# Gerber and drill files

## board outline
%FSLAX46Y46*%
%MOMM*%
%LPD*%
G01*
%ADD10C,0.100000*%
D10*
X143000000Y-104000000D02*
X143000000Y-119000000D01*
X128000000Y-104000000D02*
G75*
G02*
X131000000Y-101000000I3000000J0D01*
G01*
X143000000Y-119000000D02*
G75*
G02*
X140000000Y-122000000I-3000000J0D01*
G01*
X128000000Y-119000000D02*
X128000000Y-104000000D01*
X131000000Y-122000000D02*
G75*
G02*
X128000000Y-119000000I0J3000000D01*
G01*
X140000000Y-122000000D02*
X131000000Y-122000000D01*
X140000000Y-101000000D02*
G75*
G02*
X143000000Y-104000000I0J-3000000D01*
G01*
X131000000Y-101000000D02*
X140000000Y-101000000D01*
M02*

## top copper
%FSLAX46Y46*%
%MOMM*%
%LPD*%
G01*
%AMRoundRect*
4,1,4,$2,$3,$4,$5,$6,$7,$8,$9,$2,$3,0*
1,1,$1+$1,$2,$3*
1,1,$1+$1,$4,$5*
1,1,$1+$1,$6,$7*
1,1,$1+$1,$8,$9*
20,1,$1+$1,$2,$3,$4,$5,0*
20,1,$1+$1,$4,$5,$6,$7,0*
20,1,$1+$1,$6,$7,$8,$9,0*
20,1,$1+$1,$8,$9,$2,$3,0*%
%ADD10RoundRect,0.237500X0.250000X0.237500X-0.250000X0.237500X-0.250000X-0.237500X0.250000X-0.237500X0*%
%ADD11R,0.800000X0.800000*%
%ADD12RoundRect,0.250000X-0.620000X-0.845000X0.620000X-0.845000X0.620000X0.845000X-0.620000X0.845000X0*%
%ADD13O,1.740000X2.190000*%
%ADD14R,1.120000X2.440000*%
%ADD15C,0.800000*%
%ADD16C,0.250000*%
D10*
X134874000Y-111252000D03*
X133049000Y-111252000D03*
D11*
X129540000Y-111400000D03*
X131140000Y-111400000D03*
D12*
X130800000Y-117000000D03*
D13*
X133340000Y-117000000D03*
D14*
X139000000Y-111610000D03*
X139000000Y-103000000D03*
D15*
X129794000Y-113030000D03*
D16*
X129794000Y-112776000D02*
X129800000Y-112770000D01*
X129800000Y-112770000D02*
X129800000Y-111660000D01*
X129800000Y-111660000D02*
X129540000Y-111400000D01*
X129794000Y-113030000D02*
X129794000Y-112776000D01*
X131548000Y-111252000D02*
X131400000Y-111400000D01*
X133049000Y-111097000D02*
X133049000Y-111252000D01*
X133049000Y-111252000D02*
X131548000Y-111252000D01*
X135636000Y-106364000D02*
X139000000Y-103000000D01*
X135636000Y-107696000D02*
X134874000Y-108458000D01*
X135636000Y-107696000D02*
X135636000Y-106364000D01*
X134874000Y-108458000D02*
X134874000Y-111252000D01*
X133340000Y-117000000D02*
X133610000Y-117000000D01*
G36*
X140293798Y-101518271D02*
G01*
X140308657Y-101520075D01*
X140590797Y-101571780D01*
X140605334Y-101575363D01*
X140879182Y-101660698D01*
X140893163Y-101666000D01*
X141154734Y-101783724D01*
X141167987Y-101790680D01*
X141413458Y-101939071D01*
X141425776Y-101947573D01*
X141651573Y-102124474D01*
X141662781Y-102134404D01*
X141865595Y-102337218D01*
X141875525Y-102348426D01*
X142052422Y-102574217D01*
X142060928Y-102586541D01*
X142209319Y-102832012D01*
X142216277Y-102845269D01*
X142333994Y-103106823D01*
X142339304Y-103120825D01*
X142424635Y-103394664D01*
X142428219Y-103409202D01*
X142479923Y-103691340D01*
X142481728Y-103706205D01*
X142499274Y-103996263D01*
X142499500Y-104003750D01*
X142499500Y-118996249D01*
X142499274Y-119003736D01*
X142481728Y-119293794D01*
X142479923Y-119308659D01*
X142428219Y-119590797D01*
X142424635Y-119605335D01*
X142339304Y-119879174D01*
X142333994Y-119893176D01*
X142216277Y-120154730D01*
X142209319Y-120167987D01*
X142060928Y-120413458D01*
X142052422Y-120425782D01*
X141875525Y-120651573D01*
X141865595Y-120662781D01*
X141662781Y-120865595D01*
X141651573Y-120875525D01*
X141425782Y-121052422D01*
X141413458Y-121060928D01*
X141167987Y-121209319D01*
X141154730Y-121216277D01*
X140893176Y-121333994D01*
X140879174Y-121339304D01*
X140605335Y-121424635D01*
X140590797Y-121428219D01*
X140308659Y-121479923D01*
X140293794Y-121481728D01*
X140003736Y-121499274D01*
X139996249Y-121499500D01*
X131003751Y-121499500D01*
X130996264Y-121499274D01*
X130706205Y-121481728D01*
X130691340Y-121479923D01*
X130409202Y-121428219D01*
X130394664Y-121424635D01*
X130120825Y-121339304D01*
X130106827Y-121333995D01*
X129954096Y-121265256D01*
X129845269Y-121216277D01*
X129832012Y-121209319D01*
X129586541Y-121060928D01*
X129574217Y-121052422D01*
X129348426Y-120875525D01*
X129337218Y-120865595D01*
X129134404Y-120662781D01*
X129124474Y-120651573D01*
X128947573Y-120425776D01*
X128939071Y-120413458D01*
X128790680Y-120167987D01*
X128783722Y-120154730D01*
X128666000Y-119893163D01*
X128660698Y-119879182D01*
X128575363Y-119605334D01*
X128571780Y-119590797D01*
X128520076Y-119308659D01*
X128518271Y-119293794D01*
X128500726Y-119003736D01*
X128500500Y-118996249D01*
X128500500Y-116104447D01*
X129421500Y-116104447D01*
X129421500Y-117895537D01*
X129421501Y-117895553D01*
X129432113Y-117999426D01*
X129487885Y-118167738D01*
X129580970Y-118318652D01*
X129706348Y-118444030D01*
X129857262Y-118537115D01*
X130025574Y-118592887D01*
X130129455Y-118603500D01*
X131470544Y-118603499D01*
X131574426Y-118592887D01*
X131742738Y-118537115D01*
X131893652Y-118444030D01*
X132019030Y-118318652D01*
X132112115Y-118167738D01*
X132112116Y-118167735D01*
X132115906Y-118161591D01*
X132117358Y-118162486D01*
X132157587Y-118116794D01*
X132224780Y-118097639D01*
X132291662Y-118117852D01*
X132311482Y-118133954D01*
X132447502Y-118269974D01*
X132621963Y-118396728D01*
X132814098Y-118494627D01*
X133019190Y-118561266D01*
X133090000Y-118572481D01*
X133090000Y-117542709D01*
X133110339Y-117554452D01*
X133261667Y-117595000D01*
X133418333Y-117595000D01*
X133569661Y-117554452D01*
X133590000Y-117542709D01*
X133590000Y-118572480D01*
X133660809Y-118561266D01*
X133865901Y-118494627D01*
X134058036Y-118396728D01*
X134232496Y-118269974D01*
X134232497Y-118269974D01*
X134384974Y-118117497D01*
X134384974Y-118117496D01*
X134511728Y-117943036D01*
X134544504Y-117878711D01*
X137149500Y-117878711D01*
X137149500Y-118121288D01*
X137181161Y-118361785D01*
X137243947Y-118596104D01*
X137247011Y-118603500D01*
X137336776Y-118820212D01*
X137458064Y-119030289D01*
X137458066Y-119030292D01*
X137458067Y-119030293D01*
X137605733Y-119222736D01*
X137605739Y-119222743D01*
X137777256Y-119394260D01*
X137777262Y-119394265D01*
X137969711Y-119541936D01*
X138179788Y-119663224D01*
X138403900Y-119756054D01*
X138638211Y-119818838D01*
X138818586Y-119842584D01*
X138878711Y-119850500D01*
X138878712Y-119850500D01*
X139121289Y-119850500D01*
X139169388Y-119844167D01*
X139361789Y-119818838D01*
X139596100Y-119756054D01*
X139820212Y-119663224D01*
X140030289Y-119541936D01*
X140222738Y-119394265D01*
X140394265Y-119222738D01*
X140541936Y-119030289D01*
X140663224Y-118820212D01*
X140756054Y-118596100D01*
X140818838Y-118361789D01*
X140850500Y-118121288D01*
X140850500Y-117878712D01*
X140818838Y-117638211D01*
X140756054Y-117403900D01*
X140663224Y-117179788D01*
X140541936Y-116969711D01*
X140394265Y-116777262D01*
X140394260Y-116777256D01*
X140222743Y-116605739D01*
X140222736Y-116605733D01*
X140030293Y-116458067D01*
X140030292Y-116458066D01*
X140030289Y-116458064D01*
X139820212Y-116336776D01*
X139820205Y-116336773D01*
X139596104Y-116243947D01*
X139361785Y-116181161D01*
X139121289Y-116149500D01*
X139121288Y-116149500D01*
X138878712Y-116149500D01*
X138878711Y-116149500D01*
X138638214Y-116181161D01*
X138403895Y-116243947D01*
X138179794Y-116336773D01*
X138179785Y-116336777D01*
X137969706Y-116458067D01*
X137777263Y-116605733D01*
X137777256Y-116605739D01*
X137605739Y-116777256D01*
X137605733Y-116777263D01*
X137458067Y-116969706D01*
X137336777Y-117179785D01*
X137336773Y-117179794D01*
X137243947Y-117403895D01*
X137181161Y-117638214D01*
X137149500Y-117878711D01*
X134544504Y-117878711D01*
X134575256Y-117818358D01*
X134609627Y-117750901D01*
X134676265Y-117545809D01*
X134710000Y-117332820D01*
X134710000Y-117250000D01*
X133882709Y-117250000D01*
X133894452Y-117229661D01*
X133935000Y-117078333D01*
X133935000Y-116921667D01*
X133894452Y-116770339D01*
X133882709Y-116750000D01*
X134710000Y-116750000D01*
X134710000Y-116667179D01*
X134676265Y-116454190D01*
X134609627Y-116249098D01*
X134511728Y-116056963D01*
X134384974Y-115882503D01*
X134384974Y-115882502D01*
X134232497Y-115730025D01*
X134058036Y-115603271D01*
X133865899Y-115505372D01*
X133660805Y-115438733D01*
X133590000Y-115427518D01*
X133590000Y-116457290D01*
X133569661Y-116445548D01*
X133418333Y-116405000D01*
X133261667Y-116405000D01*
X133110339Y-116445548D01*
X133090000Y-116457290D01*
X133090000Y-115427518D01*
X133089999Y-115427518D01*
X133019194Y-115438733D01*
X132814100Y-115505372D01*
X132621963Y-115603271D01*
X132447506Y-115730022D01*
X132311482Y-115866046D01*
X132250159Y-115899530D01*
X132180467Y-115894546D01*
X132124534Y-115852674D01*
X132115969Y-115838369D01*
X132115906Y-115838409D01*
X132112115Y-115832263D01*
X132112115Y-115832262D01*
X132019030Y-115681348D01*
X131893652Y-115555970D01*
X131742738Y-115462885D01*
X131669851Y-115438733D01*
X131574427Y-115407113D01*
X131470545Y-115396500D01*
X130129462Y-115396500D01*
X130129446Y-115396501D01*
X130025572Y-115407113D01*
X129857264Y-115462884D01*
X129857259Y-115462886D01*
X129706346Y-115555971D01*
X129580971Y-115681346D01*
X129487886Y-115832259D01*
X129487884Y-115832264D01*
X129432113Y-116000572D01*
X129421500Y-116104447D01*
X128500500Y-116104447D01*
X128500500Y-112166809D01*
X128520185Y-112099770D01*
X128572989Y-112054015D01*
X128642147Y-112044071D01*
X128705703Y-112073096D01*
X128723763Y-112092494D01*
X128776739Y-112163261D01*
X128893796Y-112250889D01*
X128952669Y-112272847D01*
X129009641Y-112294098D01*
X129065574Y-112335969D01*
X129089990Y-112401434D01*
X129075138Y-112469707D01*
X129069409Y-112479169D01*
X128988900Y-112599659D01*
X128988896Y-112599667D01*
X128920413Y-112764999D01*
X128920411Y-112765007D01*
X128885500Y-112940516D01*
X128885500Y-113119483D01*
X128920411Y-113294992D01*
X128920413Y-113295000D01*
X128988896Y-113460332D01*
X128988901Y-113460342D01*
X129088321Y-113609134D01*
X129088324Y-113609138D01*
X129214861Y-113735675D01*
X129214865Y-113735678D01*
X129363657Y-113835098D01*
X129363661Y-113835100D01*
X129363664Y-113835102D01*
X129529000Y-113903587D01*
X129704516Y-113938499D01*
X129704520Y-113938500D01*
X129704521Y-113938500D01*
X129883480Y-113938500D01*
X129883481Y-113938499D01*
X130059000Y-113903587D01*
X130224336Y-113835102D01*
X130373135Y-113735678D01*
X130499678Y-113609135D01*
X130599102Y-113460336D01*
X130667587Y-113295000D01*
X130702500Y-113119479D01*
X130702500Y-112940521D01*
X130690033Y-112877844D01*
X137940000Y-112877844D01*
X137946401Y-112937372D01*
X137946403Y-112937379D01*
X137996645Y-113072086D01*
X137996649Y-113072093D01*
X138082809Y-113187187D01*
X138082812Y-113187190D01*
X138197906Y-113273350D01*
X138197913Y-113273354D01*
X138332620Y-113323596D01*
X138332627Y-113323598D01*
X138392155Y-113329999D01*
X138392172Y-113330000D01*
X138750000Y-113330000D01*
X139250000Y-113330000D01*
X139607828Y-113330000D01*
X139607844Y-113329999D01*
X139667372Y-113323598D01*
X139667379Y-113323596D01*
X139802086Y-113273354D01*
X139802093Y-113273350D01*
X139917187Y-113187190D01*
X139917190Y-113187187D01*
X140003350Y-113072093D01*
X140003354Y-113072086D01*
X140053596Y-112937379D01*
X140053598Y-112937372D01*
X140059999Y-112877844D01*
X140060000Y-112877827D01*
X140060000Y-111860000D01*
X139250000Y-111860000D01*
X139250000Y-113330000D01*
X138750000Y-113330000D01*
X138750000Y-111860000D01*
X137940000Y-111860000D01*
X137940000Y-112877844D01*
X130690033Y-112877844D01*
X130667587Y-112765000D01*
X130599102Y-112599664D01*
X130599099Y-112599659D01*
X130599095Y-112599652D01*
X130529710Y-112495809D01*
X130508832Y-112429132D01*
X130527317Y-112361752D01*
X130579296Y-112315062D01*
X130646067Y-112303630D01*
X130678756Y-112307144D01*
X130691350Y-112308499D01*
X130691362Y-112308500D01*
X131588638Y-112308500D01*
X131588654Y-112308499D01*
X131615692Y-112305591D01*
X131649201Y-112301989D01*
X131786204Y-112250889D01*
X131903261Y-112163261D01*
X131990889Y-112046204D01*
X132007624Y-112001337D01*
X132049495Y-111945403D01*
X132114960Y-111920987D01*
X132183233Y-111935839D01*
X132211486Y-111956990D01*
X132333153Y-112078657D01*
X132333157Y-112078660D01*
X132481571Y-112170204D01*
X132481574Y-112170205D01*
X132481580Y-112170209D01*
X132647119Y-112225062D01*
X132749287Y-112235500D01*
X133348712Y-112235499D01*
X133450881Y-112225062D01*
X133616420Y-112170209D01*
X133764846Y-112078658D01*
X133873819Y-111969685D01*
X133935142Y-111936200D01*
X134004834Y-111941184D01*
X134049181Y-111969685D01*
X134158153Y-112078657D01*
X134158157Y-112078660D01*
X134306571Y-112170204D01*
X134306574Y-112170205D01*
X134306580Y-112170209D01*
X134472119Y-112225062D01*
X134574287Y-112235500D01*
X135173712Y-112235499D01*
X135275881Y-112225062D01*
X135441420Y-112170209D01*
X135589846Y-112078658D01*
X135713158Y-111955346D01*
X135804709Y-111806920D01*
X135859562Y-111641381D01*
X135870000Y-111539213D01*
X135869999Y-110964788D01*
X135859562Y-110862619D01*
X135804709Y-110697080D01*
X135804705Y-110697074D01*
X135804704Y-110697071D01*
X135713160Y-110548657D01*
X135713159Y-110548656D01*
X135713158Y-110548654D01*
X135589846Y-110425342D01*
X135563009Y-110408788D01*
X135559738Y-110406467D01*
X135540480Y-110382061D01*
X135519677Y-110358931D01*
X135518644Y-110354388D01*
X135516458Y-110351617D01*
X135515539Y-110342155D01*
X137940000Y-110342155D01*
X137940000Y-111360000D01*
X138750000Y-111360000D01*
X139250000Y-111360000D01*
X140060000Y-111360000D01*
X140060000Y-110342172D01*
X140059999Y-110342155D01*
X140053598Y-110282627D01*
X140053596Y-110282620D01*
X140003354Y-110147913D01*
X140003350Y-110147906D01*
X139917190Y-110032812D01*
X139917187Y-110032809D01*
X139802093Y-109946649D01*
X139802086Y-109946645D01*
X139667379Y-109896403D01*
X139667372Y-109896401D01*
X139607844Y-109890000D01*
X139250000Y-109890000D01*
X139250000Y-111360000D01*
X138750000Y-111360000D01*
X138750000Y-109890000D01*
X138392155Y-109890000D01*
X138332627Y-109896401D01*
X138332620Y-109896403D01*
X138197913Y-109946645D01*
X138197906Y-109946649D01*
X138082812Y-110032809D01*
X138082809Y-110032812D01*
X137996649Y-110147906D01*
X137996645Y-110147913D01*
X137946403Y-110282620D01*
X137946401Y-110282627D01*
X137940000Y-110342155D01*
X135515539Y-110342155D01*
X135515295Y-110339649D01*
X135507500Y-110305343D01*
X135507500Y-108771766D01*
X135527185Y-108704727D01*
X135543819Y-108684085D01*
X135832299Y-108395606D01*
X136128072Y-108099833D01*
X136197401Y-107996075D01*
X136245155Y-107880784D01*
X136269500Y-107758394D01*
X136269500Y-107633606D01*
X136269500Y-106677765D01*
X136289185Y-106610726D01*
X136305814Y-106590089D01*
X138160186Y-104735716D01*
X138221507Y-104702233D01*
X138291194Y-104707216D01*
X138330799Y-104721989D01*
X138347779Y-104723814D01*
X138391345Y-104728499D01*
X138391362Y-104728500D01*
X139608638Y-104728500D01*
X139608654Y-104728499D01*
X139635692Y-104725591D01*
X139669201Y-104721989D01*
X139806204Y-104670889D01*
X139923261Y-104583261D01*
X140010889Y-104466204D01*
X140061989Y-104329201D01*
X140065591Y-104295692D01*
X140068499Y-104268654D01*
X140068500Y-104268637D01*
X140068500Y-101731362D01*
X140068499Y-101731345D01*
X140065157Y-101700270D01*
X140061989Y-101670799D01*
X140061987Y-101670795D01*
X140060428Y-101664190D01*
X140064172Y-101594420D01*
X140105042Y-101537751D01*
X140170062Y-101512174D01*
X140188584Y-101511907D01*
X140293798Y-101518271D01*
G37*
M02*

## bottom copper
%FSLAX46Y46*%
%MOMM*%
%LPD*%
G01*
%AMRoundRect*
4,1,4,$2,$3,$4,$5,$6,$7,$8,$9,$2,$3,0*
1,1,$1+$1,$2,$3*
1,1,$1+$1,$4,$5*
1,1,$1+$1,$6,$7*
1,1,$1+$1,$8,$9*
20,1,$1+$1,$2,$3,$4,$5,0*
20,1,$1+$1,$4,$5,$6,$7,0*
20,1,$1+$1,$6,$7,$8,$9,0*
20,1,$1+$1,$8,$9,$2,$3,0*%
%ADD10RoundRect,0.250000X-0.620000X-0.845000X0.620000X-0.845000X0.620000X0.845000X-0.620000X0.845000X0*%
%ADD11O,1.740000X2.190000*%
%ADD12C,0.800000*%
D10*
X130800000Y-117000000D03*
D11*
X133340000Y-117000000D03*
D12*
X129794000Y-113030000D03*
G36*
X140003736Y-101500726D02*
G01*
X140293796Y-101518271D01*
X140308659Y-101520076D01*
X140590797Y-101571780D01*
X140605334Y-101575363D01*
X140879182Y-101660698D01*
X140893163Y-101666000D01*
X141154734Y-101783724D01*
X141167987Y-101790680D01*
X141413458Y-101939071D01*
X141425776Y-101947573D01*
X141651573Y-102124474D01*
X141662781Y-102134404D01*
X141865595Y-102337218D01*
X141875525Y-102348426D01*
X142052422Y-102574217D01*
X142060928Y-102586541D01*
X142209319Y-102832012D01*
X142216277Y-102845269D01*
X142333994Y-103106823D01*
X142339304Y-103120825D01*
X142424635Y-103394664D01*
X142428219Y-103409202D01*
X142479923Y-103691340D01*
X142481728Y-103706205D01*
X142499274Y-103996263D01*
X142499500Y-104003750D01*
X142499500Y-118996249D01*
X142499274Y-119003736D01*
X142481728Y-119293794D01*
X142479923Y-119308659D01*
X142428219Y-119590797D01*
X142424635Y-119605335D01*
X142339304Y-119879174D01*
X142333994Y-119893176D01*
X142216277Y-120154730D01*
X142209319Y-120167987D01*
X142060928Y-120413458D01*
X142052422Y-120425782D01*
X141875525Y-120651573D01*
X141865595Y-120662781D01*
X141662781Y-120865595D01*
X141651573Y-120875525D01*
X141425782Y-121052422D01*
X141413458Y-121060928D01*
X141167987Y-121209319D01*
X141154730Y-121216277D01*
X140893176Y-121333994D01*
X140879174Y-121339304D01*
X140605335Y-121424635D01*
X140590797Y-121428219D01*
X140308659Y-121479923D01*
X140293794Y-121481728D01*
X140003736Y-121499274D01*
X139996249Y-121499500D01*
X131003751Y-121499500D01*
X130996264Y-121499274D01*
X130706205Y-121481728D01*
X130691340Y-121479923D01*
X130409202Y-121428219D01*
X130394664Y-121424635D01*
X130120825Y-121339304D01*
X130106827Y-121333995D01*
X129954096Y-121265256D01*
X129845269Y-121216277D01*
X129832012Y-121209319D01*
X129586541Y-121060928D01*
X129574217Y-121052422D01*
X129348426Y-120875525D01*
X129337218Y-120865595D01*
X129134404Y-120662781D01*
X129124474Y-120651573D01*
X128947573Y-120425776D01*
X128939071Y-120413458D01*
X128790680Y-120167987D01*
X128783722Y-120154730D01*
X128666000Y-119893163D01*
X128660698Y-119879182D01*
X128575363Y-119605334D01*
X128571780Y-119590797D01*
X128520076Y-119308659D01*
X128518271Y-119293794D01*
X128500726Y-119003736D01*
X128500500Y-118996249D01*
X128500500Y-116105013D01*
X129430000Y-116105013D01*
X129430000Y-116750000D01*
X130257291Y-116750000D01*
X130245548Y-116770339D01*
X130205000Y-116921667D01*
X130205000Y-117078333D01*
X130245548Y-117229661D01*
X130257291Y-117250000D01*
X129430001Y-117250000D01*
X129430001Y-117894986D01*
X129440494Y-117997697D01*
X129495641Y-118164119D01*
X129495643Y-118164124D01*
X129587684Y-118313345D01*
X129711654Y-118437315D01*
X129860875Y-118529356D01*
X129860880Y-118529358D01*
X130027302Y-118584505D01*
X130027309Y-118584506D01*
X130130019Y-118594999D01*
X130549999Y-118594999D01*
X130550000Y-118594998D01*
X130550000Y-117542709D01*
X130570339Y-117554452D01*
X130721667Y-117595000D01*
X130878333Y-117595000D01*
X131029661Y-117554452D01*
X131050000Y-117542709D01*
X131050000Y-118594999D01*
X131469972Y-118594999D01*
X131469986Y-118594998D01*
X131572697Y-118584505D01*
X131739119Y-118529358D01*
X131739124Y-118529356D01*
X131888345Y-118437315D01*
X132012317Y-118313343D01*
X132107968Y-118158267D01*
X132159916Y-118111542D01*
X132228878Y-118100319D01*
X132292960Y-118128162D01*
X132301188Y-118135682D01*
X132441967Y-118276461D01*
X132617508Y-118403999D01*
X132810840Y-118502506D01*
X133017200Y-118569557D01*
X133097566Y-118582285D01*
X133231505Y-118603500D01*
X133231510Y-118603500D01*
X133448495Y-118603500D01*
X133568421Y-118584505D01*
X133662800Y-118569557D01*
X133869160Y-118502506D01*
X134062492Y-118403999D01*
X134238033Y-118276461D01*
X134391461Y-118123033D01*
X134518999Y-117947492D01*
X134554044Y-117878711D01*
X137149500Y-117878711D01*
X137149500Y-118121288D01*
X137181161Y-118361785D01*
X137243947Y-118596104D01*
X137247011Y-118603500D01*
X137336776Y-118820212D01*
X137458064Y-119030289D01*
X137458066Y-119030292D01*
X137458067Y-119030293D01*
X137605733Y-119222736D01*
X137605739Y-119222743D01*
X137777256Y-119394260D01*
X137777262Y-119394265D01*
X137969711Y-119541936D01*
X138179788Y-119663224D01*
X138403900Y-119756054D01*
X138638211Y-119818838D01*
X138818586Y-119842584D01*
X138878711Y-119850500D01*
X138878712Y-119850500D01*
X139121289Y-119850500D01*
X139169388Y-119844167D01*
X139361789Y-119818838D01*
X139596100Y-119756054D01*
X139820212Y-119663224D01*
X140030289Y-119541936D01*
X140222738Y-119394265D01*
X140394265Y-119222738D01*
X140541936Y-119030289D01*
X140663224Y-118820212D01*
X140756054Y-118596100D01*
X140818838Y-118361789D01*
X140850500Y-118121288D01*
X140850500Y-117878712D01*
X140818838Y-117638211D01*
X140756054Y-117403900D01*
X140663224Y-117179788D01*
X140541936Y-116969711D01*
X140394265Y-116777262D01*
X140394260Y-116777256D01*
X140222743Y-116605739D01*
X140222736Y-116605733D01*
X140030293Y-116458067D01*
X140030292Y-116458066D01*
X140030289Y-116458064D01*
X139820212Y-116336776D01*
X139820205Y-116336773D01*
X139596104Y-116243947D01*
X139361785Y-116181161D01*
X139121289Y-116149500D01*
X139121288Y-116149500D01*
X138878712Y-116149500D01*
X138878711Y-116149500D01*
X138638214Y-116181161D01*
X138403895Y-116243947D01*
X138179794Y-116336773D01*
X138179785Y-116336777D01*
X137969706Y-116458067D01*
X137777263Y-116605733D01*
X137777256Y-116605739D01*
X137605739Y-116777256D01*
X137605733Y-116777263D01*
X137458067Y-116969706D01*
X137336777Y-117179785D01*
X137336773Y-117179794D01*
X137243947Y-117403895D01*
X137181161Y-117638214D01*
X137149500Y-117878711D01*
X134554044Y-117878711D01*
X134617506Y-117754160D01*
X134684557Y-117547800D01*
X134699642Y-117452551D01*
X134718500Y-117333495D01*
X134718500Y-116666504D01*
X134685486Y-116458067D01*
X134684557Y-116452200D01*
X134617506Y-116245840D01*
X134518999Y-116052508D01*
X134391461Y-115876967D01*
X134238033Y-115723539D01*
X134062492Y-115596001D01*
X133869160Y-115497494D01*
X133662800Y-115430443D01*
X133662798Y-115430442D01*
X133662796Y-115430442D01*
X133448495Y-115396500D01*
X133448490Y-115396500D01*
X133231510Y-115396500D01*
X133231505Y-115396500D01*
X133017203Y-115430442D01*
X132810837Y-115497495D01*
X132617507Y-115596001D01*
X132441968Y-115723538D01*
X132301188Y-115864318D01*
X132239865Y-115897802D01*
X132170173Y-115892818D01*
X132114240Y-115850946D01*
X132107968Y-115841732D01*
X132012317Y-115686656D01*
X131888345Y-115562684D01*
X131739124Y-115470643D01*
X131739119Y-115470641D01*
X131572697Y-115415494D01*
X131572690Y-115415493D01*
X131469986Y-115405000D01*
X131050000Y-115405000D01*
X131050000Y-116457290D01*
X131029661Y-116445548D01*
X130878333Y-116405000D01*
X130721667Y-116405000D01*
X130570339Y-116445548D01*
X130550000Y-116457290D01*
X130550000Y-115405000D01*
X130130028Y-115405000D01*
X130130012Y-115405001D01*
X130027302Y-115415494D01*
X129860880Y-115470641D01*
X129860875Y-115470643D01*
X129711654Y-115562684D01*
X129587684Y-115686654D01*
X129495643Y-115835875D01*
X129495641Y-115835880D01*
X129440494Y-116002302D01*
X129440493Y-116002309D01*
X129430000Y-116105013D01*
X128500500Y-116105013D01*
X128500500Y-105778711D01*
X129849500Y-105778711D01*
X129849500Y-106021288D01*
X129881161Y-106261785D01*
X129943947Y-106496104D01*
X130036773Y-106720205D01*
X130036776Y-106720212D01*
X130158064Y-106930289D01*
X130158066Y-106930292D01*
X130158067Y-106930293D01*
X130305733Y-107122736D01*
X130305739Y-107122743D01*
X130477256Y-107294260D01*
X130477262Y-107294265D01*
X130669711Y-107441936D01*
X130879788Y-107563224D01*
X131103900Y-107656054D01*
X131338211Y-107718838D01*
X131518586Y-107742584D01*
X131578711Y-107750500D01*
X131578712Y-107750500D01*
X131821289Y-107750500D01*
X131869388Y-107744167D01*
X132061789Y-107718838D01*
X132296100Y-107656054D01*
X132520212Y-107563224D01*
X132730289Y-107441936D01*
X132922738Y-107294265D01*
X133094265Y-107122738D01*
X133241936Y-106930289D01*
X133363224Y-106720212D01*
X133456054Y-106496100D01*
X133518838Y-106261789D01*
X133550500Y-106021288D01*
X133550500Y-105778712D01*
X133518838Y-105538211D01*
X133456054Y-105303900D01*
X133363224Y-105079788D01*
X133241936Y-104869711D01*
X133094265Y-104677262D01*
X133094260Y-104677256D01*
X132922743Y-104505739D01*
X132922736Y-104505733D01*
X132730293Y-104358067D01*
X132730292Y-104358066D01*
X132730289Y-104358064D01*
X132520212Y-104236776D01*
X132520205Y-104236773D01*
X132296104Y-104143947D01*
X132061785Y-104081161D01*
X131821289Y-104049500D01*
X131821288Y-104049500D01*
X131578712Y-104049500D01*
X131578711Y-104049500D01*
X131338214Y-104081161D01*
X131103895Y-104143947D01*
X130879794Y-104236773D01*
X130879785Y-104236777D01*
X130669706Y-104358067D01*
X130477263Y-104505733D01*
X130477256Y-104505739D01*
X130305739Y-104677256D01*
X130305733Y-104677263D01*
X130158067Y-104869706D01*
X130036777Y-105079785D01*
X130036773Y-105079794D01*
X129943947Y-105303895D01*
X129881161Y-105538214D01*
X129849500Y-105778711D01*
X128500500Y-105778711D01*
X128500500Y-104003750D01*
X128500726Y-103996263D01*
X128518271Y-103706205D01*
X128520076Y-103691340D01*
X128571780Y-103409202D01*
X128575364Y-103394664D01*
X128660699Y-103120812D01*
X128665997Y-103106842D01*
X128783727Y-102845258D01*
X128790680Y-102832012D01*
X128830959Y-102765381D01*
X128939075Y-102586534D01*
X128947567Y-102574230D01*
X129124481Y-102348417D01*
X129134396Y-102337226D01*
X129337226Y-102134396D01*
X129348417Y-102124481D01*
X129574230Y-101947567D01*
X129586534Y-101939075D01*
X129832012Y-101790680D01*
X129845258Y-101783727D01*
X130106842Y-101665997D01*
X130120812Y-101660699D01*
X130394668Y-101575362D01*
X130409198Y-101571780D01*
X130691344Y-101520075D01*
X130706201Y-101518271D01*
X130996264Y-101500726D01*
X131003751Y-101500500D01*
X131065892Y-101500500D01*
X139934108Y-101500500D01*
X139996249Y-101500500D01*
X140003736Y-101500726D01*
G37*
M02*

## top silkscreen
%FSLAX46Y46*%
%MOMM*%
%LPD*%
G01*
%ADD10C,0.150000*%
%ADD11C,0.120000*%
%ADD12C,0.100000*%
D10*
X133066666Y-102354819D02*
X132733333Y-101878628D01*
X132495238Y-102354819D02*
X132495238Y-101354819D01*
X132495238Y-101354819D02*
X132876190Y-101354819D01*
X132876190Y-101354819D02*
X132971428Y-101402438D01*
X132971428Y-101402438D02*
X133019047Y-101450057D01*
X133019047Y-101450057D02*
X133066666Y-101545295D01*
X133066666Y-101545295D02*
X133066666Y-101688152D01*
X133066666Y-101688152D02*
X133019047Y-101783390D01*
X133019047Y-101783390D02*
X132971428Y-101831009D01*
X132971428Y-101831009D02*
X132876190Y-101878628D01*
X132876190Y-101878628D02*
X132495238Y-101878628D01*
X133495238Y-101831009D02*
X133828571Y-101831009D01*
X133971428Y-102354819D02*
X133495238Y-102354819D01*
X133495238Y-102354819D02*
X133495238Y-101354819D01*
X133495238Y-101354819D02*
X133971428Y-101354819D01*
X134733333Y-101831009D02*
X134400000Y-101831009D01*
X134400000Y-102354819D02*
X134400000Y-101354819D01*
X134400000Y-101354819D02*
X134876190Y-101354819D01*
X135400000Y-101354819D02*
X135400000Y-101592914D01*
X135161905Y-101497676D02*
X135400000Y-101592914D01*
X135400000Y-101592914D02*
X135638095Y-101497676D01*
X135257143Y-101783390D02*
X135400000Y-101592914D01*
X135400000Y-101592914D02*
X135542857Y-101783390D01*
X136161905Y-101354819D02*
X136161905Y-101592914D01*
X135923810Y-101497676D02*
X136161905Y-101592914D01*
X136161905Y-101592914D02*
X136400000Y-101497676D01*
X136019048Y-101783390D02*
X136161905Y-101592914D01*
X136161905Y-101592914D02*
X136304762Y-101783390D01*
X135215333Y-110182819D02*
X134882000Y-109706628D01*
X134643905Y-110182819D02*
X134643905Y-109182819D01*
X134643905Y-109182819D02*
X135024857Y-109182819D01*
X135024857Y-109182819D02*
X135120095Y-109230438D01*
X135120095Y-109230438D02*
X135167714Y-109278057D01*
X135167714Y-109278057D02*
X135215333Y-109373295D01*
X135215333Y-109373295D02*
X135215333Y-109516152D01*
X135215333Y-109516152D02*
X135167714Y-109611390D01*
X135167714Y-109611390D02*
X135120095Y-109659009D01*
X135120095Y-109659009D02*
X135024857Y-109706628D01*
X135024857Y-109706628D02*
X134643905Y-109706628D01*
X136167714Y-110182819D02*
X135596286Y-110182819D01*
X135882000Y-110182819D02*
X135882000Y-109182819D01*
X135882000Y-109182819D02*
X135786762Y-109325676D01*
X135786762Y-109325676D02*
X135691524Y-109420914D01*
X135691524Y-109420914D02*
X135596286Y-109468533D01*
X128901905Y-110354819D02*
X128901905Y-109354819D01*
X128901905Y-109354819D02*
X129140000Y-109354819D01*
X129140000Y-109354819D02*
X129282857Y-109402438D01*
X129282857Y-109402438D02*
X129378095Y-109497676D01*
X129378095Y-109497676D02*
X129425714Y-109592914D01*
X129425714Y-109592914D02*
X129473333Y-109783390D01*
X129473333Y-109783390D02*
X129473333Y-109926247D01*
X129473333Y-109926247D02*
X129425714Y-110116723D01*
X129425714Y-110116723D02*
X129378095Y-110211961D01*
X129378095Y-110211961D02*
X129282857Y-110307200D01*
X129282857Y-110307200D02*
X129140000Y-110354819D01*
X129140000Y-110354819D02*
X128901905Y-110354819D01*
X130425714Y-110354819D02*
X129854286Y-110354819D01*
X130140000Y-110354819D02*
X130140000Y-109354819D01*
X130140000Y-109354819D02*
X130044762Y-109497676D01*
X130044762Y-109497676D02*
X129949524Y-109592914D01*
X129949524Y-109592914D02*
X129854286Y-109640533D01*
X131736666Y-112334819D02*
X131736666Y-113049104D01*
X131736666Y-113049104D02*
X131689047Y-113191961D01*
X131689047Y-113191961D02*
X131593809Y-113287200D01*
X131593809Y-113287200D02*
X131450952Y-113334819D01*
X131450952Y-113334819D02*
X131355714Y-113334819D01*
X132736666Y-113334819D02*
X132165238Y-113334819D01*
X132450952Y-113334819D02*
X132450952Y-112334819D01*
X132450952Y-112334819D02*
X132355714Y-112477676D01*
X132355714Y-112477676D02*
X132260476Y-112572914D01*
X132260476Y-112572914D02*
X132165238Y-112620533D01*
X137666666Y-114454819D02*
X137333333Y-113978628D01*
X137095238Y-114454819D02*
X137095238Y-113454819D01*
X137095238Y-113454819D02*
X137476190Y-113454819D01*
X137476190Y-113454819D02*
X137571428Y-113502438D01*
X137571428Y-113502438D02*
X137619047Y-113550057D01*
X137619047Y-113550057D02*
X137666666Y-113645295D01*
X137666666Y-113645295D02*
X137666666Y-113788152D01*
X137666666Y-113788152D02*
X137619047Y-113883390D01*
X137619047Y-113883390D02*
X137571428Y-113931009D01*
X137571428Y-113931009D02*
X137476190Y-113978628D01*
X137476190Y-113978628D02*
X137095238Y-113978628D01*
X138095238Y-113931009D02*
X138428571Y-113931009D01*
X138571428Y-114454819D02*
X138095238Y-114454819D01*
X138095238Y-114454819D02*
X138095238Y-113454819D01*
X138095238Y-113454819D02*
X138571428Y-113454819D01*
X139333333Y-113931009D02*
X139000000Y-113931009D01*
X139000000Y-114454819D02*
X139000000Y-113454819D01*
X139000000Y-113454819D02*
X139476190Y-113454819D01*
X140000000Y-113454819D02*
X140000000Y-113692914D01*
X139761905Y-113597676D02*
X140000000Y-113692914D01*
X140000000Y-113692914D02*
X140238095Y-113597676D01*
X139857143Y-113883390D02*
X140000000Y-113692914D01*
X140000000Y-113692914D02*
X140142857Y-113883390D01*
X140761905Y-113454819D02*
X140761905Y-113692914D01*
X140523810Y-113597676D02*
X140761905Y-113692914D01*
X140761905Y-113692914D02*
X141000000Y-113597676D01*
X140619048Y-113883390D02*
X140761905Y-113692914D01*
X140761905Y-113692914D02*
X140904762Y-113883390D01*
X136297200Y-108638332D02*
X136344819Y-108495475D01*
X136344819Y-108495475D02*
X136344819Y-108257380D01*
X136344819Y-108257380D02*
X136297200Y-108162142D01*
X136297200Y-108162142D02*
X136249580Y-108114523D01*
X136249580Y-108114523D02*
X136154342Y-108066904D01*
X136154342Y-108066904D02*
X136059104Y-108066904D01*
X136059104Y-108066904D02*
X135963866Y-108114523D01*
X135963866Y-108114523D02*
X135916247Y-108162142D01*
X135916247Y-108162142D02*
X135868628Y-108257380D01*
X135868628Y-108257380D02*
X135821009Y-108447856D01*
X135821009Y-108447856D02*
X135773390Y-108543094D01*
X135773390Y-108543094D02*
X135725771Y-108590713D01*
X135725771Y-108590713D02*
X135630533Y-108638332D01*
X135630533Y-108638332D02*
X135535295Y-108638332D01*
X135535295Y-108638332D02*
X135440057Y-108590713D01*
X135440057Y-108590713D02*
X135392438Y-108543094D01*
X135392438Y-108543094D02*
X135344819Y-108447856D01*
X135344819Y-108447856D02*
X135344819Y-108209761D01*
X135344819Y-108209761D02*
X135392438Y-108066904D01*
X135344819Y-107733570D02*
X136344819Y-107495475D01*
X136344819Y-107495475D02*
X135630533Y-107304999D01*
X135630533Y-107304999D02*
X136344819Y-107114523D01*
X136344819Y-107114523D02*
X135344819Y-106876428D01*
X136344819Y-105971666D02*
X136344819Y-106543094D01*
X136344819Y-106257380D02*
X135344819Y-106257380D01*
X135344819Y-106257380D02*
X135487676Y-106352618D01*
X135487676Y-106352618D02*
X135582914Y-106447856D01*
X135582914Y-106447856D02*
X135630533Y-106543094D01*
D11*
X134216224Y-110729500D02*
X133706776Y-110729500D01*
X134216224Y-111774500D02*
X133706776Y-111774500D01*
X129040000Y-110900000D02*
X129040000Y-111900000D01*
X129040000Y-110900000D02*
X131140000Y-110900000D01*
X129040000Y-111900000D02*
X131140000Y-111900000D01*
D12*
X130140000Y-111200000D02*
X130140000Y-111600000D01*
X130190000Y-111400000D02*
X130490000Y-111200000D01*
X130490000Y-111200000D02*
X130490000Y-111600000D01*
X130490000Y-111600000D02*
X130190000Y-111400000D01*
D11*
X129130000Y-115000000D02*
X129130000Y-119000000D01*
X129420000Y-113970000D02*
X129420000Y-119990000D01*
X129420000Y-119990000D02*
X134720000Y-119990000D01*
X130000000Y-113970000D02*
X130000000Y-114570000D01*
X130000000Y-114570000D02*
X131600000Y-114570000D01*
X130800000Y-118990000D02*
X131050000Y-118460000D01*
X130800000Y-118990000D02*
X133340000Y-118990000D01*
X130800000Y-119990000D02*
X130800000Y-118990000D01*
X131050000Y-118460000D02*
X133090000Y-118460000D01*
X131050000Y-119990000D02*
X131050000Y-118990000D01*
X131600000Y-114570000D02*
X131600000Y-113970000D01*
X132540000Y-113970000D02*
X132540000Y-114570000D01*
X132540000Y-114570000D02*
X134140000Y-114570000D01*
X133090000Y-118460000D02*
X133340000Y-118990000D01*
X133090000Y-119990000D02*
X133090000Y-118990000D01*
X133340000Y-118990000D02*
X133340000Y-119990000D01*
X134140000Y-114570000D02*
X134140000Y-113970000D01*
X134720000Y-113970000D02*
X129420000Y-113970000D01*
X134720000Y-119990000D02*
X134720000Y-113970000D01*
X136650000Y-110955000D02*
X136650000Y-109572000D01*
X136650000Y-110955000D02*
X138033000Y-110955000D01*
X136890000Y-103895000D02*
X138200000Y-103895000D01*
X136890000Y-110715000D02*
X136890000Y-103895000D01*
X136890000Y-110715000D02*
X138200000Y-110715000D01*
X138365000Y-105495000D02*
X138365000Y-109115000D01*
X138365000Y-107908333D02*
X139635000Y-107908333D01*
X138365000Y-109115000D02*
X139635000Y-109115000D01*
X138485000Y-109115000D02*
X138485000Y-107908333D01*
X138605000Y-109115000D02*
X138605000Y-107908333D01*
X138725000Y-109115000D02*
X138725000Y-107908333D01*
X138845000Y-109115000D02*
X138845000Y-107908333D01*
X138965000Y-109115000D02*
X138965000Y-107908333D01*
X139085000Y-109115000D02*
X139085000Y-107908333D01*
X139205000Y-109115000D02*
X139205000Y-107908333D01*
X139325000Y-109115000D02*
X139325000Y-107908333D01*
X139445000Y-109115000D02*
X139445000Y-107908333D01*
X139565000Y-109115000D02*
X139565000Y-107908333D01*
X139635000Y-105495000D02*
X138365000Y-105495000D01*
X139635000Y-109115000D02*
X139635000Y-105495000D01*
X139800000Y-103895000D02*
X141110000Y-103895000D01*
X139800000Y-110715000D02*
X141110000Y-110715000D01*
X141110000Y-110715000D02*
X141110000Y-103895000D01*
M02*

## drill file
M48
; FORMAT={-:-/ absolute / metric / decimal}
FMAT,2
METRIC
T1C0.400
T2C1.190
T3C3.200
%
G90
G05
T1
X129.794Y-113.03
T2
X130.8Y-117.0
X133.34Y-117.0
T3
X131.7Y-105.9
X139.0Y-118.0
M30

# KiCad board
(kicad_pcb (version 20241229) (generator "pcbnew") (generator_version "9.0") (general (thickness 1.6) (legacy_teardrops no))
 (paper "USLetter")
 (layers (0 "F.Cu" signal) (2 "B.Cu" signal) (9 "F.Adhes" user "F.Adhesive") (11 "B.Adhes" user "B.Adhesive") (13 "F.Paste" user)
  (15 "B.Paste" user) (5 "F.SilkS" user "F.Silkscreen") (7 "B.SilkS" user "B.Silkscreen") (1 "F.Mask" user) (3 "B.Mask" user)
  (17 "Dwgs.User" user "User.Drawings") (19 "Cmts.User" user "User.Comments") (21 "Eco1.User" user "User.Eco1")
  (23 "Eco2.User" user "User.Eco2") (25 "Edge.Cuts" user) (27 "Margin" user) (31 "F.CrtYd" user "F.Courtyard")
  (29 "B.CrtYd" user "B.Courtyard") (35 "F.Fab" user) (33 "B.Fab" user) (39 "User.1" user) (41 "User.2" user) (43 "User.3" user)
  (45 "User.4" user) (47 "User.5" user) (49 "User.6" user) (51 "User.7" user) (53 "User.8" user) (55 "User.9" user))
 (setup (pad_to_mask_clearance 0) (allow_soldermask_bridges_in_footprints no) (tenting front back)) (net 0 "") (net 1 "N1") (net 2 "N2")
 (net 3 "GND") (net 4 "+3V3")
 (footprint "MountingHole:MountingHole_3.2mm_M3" (layer "F.Cu") (at 131.7 105.9)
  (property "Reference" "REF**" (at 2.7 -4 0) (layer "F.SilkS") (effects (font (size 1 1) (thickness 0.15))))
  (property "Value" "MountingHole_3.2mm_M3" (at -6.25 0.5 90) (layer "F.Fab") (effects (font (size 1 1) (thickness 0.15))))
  (pad "" np_thru_hole circle (at 0 0) (size 3.2 3.2) (drill 3.2) (layers "*.Cu" "*.Mask")))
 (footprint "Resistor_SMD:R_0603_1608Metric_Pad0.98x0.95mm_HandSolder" (layer "F.Cu") (at 133.9615 111.252 180)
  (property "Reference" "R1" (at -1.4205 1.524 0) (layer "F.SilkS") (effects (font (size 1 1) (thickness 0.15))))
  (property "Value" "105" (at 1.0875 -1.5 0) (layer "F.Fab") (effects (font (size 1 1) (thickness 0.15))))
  (fp_line (start -0.254724 0.5225) (end 0.254724 0.5225) (stroke (width 0.12) (type solid)) (layer "F.SilkS"))
  (fp_line (start -0.254724 -0.5225) (end 0.254724 -0.5225) (stroke (width 0.12) (type solid)) (layer "F.SilkS"))
  (pad "1" smd roundrect (at -0.9125 0 180) (size 0.975 0.95) (layers "F.Cu" "F.Mask" "F.Paste") (roundrect_rratio 0.25) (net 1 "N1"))
  (pad "2" smd roundrect (at 0.9125 0 180) (size 0.975 0.95) (layers "F.Cu" "F.Mask" "F.Paste") (roundrect_rratio 0.25) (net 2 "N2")))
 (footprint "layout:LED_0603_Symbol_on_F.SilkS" (layer "F.Cu") (at 130.34 111.4)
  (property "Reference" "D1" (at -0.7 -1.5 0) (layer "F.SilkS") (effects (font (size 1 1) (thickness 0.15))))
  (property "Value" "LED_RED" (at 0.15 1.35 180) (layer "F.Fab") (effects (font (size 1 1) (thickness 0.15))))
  (fp_line (start -1.3 -0.5) (end -1.3 0.5) (stroke (width 0.12) (type solid)) (layer "F.SilkS"))
  (fp_line (start -1.3 -0.5) (end 0.8 -0.5) (stroke (width 0.12) (type solid)) (layer "F.SilkS"))
  (fp_line (start -1.3 0.5) (end 0.8 0.5) (stroke (width 0.12) (type solid)) (layer "F.SilkS"))
  (fp_line (start -0.2 -0.2) (end -0.2 0.2) (stroke (width 0.1) (type solid)) (layer "F.SilkS"))
  (fp_line (start -0.15 0) (end 0.15 -0.2) (stroke (width 0.1) (type solid)) (layer "F.SilkS"))
  (fp_line (start 0.15 -0.2) (end 0.15 0.2) (stroke (width 0.1) (type solid)) (layer "F.SilkS"))
  (fp_line (start 0.15 0.2) (end -0.15 0) (stroke (width 0.1) (type solid)) (layer "F.SilkS"))
  (pad "1" smd rect (at -0.8 0 180) (size 0.8 0.8) (layers "F.Cu" "F.Mask" "F.Paste") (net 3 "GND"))
  (pad "2" smd rect (at 0.8 0 180) (size 0.8 0.8) (layers "F.Cu" "F.Mask" "F.Paste") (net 2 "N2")))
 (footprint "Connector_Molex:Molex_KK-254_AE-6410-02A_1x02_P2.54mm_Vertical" (layer "F.Cu") (at 130.8 117)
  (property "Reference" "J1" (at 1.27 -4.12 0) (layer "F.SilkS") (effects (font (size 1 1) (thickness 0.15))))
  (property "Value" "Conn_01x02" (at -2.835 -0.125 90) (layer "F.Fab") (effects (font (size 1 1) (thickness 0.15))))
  (fp_line (start -1.67 -2) (end -1.67 2) (stroke (width 0.12) (type solid)) (layer "F.SilkS"))
  (fp_line (start -1.38 -3.03) (end -1.38 2.99) (stroke (width 0.12) (type solid)) (layer "F.SilkS"))
  (fp_line (start -1.38 2.99) (end 3.92 2.99) (stroke (width 0.12) (type solid)) (layer "F.SilkS"))
  (fp_line (start -0.8 -3.03) (end -0.8 -2.43) (stroke (width 0.12) (type solid)) (layer "F.SilkS"))
  (fp_line (start -0.8 -2.43) (end 0.8 -2.43) (stroke (width 0.12) (type solid)) (layer "F.SilkS"))
  (fp_line (start 0 1.99) (end 0.25 1.46) (stroke (width 0.12) (type solid)) (layer "F.SilkS"))
  (fp_line (start 0 1.99) (end 2.54 1.99) (stroke (width 0.12) (type solid)) (layer "F.SilkS"))
  (fp_line (start 0 2.99) (end 0 1.99) (stroke (width 0.12) (type solid)) (layer "F.SilkS"))
  (fp_line (start 0.25 1.46) (end 2.29 1.46) (stroke (width 0.12) (type solid)) (layer "F.SilkS"))
  (fp_line (start 0.25 2.99) (end 0.25 1.99) (stroke (width 0.12) (type solid)) (layer "F.SilkS"))
  (fp_line (start 0.8 -2.43) (end 0.8 -3.03) (stroke (width 0.12) (type solid)) (layer "F.SilkS"))
  (fp_line (start 1.74 -3.03) (end 1.74 -2.43) (stroke (width 0.12) (type solid)) (layer "F.SilkS"))
  (fp_line (start 1.74 -2.43) (end 3.34 -2.43) (stroke (width 0.12) (type solid)) (layer "F.SilkS"))
  (fp_line (start 2.29 1.46) (end 2.54 1.99) (stroke (width 0.12) (type solid)) (layer "F.SilkS"))
  (fp_line (start 2.29 2.99) (end 2.29 1.99) (stroke (width 0.12) (type solid)) (layer "F.SilkS"))
  (fp_line (start 2.54 1.99) (end 2.54 2.99) (stroke (width 0.12) (type solid)) (layer "F.SilkS"))
  (fp_line (start 3.34 -2.43) (end 3.34 -3.03) (stroke (width 0.12) (type solid)) (layer "F.SilkS"))
  (fp_line (start 3.92 -3.03) (end -1.38 -3.03) (stroke (width 0.12) (type solid)) (layer "F.SilkS"))
  (fp_line (start 3.92 2.99) (end 3.92 -3.03) (stroke (width 0.12) (type solid)) (layer "F.SilkS"))
  (pad "1" thru_hole roundrect (at 0 0) (size 1.74 2.19) (drill 1.19) (layers "*.Cu" "*.Mask") (remove_unused_layers no)
   (roundrect_rratio 0.143678) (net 3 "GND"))
  (pad "2" thru_hole oval (at 2.54 0) (size 1.74 2.19) (drill 1.19) (layers "*.Cu" "*.Mask") (remove_unused_layers no) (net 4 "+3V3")))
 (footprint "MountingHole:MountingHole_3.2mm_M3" (layer "F.Cu") (at 139 118)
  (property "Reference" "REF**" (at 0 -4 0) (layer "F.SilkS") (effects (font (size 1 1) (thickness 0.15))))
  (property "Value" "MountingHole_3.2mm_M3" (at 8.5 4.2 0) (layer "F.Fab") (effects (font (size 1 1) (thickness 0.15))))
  (pad "" np_thru_hole circle (at 0 0) (size 3.2 3.2) (drill 3.2) (layers "*.Cu" "*.Mask")))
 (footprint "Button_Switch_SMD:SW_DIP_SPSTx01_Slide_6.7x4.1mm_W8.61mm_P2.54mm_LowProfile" (layer "F.Cu") (at 139 107.305 90)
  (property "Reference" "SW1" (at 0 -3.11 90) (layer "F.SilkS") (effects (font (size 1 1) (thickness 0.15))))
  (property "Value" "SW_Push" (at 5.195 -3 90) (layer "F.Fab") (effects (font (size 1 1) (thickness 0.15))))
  (fp_line (start -3.65 -2.35) (end -2.267 -2.35) (stroke (width 0.12) (type solid)) (layer "F.SilkS"))
  (fp_line (start -3.65 -2.35) (end -3.65 -0.967) (stroke (width 0.12) (type solid)) (layer "F.SilkS"))
  (fp_line (start 3.41 -2.11) (end 3.41 -0.8) (stroke (width 0.12) (type solid)) (layer "F.SilkS"))
  (fp_line (start -3.41 -2.11) (end 3.41 -2.11) (stroke (width 0.12) (type solid)) (layer "F.SilkS"))
  (fp_line (start -3.41 -2.11) (end -3.41 -0.8) (stroke (width 0.12) (type solid)) (layer "F.SilkS"))
  (fp_line (start 1.81 -0.635) (end -1.81 -0.635) (stroke (width 0.12) (type solid)) (layer "F.SilkS"))
  (fp_line (start -0.603333 -0.635) (end -0.603333 0.635) (stroke (width 0.12) (type solid)) (layer "F.SilkS"))
  (fp_line (start -1.81 -0.635) (end -1.81 0.635) (stroke (width 0.12) (type solid)) (layer "F.SilkS"))
  (fp_line (start -1.81 -0.515) (end -0.603333 -0.515) (stroke (width 0.12) (type solid)) (layer "F.SilkS"))
  (fp_line (start -1.81 -0.395) (end -0.603333 -0.395) (stroke (width 0.12) (type solid)) (layer "F.SilkS"))
  (fp_line (start -1.81 -0.275) (end -0.603333 -0.275) (stroke (width 0.12) (type solid)) (layer "F.SilkS"))
  (fp_line (start -1.81 -0.155) (end -0.603333 -0.155) (stroke (width 0.12) (type solid)) (layer "F.SilkS"))
  (fp_line (start -1.81 -0.035) (end -0.603333 -0.035) (stroke (width 0.12) (type solid)) (layer "F.SilkS"))
  (fp_line (start -1.81 0.085) (end -0.603333 0.085) (stroke (width 0.12) (type solid)) (layer "F.SilkS"))
  (fp_line (start -1.81 0.205) (end -0.603333 0.205) (stroke (width 0.12) (type solid)) (layer "F.SilkS"))
  (fp_line (start -1.81 0.325) (end -0.603333 0.325) (stroke (width 0.12) (type solid)) (layer "F.SilkS"))
  (fp_line (start -1.81 0.445) (end -0.603333 0.445) (stroke (width 0.12) (type solid)) (layer "F.SilkS"))
  (fp_line (start -1.81 0.565) (end -0.603333 0.565) (stroke (width 0.12) (type solid)) (layer "F.SilkS"))
  (fp_line (start 1.81 0.635) (end 1.81 -0.635) (stroke (width 0.12) (type solid)) (layer "F.SilkS"))
  (fp_line (start -1.81 0.635) (end 1.81 0.635) (stroke (width 0.12) (type solid)) (layer "F.SilkS"))
  (fp_line (start 3.41 0.8) (end 3.41 2.11) (stroke (width 0.12) (type solid)) (layer "F.SilkS"))
  (fp_line (start -3.41 0.8) (end -3.41 2.11) (stroke (width 0.12) (type solid)) (layer "F.SilkS"))
  (fp_line (start -3.41 2.11) (end 3.41 2.11) (stroke (width 0.12) (type solid)) (layer "F.SilkS"))
  (pad "1" smd rect (at -4.305 0 90) (size 2.44 1.12) (layers "F.Cu" "F.Mask" "F.Paste") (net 4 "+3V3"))
  (pad "2" smd rect (at 4.305 0 90) (size 2.44 1.12) (layers "F.Cu" "F.Mask" "F.Paste") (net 1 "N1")))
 (gr_line (start 143 104) (end 143 119) (stroke (width 0.1) (type solid)) (layer "Edge.Cuts"))
 (gr_arc (start 128 104) (mid 128.87868 101.87868) (end 131 101) (stroke (width 0.1) (type default)) (layer "Edge.Cuts"))
 (gr_arc (start 143 119) (mid 142.12132 121.12132) (end 140 122) (stroke (width 0.1) (type default)) (layer "Edge.Cuts"))
 (gr_line (start 128 119) (end 128 104) (stroke (width 0.1) (type default)) (layer "Edge.Cuts"))
 (gr_arc (start 131 122) (mid 128.87868 121.12132) (end 128 119) (stroke (width 0.1) (type default)) (layer "Edge.Cuts"))
 (gr_line (start 140 122) (end 131 122) (stroke (width 0.1) (type default)) (layer "Edge.Cuts"))
 (gr_arc (start 140 101) (mid 142.12132 101.87868) (end 143 104) (stroke (width 0.1) (type default)) (layer "Edge.Cuts"))
 (gr_line (start 131 101) (end 140 101) (stroke (width 0.1) (type default)) (layer "Edge.Cuts"))
 (segment (start 129.794 112.776) (end 129.8 112.77) (width 0.25) (layer "F.Cu") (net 3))
 (segment (start 129.8 112.77) (end 129.8 111.66) (width 0.25) (layer "F.Cu") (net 3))
 (segment (start 129.8 111.66) (end 129.54 111.4) (width 0.25) (layer "F.Cu") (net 3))
 (segment (start 129.794 113.03) (end 129.794 112.776) (width 0.25) (layer "F.Cu") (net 3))
 (via (at 129.794 113.03) (size 0.8) (drill 0.4) (layers "F.Cu" "B.Cu") (free yes) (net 3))
 (segment (start 131.548 111.252) (end 131.4 111.4) (width 0.25) (layer "F.Cu") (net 2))
 (segment (start 133.049 111.097) (end 133.049 111.252) (width 0.25) (layer "F.Cu") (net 2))
 (segment (start 133.049 111.252) (end 131.548 111.252) (width 0.25) (layer "F.Cu") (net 2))
 (segment (start 135.636 106.364) (end 139 103) (width 0.25) (layer "F.Cu") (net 1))
 (segment (start 135.636 107.696) (end 134.874 108.458) (width 0.25) (layer "F.Cu") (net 1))
 (segment (start 135.636 107.696) (end 135.636 106.364) (width 0.25) (layer "F.Cu") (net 1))
 (segment (start 134.874 108.458) (end 134.874 111.252) (width 0.25) (layer "F.Cu") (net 1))
 (segment (start 133.34 117) (end 133.61 117) (width 0.25) (layer "F.Cu") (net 4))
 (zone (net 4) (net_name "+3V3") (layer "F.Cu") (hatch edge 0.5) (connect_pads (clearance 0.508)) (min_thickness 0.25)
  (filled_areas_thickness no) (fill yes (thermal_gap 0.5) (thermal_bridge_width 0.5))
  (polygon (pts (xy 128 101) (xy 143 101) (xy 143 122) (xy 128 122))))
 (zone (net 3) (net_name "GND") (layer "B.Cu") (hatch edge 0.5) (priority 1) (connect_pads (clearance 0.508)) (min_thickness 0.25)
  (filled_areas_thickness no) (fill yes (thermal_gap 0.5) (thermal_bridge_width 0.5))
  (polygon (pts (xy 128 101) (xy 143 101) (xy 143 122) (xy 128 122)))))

